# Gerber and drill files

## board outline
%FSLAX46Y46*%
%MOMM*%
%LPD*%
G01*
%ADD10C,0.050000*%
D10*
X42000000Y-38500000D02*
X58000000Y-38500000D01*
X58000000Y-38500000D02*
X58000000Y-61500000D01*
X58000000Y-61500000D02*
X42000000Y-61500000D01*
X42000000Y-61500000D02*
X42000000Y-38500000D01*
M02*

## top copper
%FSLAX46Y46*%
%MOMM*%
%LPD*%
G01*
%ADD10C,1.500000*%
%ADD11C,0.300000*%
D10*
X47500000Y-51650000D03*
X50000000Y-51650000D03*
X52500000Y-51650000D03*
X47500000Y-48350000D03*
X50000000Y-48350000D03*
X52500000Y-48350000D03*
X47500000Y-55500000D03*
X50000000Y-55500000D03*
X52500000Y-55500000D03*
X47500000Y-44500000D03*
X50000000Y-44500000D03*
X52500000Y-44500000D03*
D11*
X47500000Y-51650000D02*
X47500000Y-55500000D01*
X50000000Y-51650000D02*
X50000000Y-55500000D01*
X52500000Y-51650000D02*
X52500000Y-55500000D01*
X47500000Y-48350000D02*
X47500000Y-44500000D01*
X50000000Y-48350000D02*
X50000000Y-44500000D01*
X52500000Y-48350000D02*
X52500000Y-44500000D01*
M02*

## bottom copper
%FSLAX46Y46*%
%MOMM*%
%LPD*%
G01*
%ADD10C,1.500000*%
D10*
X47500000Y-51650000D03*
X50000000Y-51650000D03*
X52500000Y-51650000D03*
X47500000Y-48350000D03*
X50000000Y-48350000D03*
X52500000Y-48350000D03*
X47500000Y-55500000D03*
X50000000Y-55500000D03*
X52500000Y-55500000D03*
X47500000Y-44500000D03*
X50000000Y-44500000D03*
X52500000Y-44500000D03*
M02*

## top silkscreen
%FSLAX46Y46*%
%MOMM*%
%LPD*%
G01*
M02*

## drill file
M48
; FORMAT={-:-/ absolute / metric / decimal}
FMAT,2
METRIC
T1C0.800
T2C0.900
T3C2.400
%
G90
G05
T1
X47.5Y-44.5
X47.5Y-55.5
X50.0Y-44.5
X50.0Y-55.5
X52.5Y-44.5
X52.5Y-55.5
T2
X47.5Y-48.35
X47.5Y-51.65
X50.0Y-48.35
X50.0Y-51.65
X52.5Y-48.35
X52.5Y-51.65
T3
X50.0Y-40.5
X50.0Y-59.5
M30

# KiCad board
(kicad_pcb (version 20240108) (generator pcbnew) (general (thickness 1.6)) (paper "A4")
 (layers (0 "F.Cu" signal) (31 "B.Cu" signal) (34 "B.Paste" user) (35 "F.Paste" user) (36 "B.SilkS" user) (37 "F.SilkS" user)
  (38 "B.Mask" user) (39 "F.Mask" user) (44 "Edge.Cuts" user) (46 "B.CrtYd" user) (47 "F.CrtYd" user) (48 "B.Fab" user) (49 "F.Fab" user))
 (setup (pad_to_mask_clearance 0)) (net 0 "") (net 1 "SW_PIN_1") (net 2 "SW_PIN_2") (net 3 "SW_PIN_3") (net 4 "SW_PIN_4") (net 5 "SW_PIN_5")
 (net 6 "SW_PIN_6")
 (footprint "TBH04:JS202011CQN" (layer "F.Cu") (at 50 50)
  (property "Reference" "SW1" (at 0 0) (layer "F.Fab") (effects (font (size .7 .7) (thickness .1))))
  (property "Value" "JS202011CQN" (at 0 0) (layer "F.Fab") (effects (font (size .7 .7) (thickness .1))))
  (pad "1" thru_hole circle (at -2.5 1.65) (size 1.5 1.5) (drill .9) (layers "*.Cu" "*.Mask") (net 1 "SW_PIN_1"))
  (pad "2" thru_hole circle (at 0 1.65) (size 1.5 1.5) (drill .9) (layers "*.Cu" "*.Mask") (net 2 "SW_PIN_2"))
  (pad "3" thru_hole circle (at 2.5 1.65) (size 1.5 1.5) (drill .9) (layers "*.Cu" "*.Mask") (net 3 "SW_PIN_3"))
  (pad "4" thru_hole circle (at -2.5 -1.65) (size 1.5 1.5) (drill .9) (layers "*.Cu" "*.Mask") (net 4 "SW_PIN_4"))
  (pad "5" thru_hole circle (at 0 -1.65) (size 1.5 1.5) (drill .9) (layers "*.Cu" "*.Mask") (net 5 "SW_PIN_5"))
  (pad "6" thru_hole circle (at 2.5 -1.65) (size 1.5 1.5) (drill .9) (layers "*.Cu" "*.Mask") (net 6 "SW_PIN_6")))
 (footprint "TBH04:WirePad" (layer "F.Cu") (at 47.5 55.5)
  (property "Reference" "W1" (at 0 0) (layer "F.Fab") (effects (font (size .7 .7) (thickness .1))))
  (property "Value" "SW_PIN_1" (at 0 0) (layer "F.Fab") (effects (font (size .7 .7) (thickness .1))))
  (pad "1" thru_hole circle (at 0 0) (size 1.5 1.5) (drill .8) (layers "*.Cu" "*.Mask") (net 1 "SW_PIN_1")))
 (segment (start 47.5 51.65) (end 47.5 55.5) (width .3) (layer "F.Cu") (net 1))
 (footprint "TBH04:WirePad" (layer "F.Cu") (at 50 55.5)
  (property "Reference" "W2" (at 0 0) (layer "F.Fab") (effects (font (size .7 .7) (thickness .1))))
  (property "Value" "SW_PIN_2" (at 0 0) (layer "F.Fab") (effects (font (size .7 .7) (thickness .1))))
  (pad "1" thru_hole circle (at 0 0) (size 1.5 1.5) (drill .8) (layers "*.Cu" "*.Mask") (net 2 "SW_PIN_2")))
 (segment (start 50 51.65) (end 50 55.5) (width .3) (layer "F.Cu") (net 2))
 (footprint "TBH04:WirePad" (layer "F.Cu") (at 52.5 55.5)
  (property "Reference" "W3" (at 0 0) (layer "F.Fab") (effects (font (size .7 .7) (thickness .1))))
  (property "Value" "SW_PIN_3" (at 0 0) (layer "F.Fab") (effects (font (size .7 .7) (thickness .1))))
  (pad "1" thru_hole circle (at 0 0) (size 1.5 1.5) (drill .8) (layers "*.Cu" "*.Mask") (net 3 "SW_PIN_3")))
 (segment (start 52.5 51.65) (end 52.5 55.5) (width .3) (layer "F.Cu") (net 3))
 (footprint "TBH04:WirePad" (layer "F.Cu") (at 47.5 44.5)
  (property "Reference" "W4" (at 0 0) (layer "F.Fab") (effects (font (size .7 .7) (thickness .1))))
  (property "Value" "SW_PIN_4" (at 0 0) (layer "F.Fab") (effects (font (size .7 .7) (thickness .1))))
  (pad "1" thru_hole circle (at 0 0) (size 1.5 1.5) (drill .8) (layers "*.Cu" "*.Mask") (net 4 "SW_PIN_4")))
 (segment (start 47.5 48.35) (end 47.5 44.5) (width .3) (layer "F.Cu") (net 4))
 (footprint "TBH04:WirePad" (layer "F.Cu") (at 50 44.5)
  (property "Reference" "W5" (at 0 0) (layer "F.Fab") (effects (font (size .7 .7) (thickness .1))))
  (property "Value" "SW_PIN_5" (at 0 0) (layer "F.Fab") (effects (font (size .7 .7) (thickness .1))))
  (pad "1" thru_hole circle (at 0 0) (size 1.5 1.5) (drill .8) (layers "*.Cu" "*.Mask") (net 5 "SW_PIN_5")))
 (segment (start 50 48.35) (end 50 44.5) (width .3) (layer "F.Cu") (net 5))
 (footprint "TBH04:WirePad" (layer "F.Cu") (at 52.5 44.5)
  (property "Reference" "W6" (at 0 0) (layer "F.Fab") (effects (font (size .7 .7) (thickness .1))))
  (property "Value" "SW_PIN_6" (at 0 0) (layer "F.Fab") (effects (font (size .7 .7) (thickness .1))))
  (pad "1" thru_hole circle (at 0 0) (size 1.5 1.5) (drill .8) (layers "*.Cu" "*.Mask") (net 6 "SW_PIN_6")))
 (segment (start 52.5 48.35) (end 52.5 44.5) (width .3) (layer "F.Cu") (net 6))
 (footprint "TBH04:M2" (layer "F.Cu") (at 50 40.5)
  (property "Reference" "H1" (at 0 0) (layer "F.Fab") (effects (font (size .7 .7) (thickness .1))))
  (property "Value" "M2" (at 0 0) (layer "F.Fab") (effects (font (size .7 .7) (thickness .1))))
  (pad "" np_thru_hole circle (at 0 0) (size 2.4 2.4) (drill 2.4) (layers "*.Cu" "*.Mask")))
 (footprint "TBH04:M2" (layer "F.Cu") (at 50 59.5)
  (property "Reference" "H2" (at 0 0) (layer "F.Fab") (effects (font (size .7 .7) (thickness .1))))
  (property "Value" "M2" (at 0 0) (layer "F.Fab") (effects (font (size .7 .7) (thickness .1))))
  (pad "" np_thru_hole circle (at 0 0) (size 2.4 2.4) (drill 2.4) (layers "*.Cu" "*.Mask")))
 (gr_line (start 42 38.5) (end 58 38.5) (stroke (width .05) (type default)) (layer "Edge.Cuts"))
 (gr_line (start 58 38.5) (end 58 61.5) (stroke (width .05) (type default)) (layer "Edge.Cuts"))
 (gr_line (start 58 61.5) (end 42 61.5) (stroke (width .05) (type default)) (layer "Edge.Cuts"))
 (gr_line (start 42 61.5) (end 42 38.5) (stroke (width .05) (type default)) (layer "Edge.Cuts")))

